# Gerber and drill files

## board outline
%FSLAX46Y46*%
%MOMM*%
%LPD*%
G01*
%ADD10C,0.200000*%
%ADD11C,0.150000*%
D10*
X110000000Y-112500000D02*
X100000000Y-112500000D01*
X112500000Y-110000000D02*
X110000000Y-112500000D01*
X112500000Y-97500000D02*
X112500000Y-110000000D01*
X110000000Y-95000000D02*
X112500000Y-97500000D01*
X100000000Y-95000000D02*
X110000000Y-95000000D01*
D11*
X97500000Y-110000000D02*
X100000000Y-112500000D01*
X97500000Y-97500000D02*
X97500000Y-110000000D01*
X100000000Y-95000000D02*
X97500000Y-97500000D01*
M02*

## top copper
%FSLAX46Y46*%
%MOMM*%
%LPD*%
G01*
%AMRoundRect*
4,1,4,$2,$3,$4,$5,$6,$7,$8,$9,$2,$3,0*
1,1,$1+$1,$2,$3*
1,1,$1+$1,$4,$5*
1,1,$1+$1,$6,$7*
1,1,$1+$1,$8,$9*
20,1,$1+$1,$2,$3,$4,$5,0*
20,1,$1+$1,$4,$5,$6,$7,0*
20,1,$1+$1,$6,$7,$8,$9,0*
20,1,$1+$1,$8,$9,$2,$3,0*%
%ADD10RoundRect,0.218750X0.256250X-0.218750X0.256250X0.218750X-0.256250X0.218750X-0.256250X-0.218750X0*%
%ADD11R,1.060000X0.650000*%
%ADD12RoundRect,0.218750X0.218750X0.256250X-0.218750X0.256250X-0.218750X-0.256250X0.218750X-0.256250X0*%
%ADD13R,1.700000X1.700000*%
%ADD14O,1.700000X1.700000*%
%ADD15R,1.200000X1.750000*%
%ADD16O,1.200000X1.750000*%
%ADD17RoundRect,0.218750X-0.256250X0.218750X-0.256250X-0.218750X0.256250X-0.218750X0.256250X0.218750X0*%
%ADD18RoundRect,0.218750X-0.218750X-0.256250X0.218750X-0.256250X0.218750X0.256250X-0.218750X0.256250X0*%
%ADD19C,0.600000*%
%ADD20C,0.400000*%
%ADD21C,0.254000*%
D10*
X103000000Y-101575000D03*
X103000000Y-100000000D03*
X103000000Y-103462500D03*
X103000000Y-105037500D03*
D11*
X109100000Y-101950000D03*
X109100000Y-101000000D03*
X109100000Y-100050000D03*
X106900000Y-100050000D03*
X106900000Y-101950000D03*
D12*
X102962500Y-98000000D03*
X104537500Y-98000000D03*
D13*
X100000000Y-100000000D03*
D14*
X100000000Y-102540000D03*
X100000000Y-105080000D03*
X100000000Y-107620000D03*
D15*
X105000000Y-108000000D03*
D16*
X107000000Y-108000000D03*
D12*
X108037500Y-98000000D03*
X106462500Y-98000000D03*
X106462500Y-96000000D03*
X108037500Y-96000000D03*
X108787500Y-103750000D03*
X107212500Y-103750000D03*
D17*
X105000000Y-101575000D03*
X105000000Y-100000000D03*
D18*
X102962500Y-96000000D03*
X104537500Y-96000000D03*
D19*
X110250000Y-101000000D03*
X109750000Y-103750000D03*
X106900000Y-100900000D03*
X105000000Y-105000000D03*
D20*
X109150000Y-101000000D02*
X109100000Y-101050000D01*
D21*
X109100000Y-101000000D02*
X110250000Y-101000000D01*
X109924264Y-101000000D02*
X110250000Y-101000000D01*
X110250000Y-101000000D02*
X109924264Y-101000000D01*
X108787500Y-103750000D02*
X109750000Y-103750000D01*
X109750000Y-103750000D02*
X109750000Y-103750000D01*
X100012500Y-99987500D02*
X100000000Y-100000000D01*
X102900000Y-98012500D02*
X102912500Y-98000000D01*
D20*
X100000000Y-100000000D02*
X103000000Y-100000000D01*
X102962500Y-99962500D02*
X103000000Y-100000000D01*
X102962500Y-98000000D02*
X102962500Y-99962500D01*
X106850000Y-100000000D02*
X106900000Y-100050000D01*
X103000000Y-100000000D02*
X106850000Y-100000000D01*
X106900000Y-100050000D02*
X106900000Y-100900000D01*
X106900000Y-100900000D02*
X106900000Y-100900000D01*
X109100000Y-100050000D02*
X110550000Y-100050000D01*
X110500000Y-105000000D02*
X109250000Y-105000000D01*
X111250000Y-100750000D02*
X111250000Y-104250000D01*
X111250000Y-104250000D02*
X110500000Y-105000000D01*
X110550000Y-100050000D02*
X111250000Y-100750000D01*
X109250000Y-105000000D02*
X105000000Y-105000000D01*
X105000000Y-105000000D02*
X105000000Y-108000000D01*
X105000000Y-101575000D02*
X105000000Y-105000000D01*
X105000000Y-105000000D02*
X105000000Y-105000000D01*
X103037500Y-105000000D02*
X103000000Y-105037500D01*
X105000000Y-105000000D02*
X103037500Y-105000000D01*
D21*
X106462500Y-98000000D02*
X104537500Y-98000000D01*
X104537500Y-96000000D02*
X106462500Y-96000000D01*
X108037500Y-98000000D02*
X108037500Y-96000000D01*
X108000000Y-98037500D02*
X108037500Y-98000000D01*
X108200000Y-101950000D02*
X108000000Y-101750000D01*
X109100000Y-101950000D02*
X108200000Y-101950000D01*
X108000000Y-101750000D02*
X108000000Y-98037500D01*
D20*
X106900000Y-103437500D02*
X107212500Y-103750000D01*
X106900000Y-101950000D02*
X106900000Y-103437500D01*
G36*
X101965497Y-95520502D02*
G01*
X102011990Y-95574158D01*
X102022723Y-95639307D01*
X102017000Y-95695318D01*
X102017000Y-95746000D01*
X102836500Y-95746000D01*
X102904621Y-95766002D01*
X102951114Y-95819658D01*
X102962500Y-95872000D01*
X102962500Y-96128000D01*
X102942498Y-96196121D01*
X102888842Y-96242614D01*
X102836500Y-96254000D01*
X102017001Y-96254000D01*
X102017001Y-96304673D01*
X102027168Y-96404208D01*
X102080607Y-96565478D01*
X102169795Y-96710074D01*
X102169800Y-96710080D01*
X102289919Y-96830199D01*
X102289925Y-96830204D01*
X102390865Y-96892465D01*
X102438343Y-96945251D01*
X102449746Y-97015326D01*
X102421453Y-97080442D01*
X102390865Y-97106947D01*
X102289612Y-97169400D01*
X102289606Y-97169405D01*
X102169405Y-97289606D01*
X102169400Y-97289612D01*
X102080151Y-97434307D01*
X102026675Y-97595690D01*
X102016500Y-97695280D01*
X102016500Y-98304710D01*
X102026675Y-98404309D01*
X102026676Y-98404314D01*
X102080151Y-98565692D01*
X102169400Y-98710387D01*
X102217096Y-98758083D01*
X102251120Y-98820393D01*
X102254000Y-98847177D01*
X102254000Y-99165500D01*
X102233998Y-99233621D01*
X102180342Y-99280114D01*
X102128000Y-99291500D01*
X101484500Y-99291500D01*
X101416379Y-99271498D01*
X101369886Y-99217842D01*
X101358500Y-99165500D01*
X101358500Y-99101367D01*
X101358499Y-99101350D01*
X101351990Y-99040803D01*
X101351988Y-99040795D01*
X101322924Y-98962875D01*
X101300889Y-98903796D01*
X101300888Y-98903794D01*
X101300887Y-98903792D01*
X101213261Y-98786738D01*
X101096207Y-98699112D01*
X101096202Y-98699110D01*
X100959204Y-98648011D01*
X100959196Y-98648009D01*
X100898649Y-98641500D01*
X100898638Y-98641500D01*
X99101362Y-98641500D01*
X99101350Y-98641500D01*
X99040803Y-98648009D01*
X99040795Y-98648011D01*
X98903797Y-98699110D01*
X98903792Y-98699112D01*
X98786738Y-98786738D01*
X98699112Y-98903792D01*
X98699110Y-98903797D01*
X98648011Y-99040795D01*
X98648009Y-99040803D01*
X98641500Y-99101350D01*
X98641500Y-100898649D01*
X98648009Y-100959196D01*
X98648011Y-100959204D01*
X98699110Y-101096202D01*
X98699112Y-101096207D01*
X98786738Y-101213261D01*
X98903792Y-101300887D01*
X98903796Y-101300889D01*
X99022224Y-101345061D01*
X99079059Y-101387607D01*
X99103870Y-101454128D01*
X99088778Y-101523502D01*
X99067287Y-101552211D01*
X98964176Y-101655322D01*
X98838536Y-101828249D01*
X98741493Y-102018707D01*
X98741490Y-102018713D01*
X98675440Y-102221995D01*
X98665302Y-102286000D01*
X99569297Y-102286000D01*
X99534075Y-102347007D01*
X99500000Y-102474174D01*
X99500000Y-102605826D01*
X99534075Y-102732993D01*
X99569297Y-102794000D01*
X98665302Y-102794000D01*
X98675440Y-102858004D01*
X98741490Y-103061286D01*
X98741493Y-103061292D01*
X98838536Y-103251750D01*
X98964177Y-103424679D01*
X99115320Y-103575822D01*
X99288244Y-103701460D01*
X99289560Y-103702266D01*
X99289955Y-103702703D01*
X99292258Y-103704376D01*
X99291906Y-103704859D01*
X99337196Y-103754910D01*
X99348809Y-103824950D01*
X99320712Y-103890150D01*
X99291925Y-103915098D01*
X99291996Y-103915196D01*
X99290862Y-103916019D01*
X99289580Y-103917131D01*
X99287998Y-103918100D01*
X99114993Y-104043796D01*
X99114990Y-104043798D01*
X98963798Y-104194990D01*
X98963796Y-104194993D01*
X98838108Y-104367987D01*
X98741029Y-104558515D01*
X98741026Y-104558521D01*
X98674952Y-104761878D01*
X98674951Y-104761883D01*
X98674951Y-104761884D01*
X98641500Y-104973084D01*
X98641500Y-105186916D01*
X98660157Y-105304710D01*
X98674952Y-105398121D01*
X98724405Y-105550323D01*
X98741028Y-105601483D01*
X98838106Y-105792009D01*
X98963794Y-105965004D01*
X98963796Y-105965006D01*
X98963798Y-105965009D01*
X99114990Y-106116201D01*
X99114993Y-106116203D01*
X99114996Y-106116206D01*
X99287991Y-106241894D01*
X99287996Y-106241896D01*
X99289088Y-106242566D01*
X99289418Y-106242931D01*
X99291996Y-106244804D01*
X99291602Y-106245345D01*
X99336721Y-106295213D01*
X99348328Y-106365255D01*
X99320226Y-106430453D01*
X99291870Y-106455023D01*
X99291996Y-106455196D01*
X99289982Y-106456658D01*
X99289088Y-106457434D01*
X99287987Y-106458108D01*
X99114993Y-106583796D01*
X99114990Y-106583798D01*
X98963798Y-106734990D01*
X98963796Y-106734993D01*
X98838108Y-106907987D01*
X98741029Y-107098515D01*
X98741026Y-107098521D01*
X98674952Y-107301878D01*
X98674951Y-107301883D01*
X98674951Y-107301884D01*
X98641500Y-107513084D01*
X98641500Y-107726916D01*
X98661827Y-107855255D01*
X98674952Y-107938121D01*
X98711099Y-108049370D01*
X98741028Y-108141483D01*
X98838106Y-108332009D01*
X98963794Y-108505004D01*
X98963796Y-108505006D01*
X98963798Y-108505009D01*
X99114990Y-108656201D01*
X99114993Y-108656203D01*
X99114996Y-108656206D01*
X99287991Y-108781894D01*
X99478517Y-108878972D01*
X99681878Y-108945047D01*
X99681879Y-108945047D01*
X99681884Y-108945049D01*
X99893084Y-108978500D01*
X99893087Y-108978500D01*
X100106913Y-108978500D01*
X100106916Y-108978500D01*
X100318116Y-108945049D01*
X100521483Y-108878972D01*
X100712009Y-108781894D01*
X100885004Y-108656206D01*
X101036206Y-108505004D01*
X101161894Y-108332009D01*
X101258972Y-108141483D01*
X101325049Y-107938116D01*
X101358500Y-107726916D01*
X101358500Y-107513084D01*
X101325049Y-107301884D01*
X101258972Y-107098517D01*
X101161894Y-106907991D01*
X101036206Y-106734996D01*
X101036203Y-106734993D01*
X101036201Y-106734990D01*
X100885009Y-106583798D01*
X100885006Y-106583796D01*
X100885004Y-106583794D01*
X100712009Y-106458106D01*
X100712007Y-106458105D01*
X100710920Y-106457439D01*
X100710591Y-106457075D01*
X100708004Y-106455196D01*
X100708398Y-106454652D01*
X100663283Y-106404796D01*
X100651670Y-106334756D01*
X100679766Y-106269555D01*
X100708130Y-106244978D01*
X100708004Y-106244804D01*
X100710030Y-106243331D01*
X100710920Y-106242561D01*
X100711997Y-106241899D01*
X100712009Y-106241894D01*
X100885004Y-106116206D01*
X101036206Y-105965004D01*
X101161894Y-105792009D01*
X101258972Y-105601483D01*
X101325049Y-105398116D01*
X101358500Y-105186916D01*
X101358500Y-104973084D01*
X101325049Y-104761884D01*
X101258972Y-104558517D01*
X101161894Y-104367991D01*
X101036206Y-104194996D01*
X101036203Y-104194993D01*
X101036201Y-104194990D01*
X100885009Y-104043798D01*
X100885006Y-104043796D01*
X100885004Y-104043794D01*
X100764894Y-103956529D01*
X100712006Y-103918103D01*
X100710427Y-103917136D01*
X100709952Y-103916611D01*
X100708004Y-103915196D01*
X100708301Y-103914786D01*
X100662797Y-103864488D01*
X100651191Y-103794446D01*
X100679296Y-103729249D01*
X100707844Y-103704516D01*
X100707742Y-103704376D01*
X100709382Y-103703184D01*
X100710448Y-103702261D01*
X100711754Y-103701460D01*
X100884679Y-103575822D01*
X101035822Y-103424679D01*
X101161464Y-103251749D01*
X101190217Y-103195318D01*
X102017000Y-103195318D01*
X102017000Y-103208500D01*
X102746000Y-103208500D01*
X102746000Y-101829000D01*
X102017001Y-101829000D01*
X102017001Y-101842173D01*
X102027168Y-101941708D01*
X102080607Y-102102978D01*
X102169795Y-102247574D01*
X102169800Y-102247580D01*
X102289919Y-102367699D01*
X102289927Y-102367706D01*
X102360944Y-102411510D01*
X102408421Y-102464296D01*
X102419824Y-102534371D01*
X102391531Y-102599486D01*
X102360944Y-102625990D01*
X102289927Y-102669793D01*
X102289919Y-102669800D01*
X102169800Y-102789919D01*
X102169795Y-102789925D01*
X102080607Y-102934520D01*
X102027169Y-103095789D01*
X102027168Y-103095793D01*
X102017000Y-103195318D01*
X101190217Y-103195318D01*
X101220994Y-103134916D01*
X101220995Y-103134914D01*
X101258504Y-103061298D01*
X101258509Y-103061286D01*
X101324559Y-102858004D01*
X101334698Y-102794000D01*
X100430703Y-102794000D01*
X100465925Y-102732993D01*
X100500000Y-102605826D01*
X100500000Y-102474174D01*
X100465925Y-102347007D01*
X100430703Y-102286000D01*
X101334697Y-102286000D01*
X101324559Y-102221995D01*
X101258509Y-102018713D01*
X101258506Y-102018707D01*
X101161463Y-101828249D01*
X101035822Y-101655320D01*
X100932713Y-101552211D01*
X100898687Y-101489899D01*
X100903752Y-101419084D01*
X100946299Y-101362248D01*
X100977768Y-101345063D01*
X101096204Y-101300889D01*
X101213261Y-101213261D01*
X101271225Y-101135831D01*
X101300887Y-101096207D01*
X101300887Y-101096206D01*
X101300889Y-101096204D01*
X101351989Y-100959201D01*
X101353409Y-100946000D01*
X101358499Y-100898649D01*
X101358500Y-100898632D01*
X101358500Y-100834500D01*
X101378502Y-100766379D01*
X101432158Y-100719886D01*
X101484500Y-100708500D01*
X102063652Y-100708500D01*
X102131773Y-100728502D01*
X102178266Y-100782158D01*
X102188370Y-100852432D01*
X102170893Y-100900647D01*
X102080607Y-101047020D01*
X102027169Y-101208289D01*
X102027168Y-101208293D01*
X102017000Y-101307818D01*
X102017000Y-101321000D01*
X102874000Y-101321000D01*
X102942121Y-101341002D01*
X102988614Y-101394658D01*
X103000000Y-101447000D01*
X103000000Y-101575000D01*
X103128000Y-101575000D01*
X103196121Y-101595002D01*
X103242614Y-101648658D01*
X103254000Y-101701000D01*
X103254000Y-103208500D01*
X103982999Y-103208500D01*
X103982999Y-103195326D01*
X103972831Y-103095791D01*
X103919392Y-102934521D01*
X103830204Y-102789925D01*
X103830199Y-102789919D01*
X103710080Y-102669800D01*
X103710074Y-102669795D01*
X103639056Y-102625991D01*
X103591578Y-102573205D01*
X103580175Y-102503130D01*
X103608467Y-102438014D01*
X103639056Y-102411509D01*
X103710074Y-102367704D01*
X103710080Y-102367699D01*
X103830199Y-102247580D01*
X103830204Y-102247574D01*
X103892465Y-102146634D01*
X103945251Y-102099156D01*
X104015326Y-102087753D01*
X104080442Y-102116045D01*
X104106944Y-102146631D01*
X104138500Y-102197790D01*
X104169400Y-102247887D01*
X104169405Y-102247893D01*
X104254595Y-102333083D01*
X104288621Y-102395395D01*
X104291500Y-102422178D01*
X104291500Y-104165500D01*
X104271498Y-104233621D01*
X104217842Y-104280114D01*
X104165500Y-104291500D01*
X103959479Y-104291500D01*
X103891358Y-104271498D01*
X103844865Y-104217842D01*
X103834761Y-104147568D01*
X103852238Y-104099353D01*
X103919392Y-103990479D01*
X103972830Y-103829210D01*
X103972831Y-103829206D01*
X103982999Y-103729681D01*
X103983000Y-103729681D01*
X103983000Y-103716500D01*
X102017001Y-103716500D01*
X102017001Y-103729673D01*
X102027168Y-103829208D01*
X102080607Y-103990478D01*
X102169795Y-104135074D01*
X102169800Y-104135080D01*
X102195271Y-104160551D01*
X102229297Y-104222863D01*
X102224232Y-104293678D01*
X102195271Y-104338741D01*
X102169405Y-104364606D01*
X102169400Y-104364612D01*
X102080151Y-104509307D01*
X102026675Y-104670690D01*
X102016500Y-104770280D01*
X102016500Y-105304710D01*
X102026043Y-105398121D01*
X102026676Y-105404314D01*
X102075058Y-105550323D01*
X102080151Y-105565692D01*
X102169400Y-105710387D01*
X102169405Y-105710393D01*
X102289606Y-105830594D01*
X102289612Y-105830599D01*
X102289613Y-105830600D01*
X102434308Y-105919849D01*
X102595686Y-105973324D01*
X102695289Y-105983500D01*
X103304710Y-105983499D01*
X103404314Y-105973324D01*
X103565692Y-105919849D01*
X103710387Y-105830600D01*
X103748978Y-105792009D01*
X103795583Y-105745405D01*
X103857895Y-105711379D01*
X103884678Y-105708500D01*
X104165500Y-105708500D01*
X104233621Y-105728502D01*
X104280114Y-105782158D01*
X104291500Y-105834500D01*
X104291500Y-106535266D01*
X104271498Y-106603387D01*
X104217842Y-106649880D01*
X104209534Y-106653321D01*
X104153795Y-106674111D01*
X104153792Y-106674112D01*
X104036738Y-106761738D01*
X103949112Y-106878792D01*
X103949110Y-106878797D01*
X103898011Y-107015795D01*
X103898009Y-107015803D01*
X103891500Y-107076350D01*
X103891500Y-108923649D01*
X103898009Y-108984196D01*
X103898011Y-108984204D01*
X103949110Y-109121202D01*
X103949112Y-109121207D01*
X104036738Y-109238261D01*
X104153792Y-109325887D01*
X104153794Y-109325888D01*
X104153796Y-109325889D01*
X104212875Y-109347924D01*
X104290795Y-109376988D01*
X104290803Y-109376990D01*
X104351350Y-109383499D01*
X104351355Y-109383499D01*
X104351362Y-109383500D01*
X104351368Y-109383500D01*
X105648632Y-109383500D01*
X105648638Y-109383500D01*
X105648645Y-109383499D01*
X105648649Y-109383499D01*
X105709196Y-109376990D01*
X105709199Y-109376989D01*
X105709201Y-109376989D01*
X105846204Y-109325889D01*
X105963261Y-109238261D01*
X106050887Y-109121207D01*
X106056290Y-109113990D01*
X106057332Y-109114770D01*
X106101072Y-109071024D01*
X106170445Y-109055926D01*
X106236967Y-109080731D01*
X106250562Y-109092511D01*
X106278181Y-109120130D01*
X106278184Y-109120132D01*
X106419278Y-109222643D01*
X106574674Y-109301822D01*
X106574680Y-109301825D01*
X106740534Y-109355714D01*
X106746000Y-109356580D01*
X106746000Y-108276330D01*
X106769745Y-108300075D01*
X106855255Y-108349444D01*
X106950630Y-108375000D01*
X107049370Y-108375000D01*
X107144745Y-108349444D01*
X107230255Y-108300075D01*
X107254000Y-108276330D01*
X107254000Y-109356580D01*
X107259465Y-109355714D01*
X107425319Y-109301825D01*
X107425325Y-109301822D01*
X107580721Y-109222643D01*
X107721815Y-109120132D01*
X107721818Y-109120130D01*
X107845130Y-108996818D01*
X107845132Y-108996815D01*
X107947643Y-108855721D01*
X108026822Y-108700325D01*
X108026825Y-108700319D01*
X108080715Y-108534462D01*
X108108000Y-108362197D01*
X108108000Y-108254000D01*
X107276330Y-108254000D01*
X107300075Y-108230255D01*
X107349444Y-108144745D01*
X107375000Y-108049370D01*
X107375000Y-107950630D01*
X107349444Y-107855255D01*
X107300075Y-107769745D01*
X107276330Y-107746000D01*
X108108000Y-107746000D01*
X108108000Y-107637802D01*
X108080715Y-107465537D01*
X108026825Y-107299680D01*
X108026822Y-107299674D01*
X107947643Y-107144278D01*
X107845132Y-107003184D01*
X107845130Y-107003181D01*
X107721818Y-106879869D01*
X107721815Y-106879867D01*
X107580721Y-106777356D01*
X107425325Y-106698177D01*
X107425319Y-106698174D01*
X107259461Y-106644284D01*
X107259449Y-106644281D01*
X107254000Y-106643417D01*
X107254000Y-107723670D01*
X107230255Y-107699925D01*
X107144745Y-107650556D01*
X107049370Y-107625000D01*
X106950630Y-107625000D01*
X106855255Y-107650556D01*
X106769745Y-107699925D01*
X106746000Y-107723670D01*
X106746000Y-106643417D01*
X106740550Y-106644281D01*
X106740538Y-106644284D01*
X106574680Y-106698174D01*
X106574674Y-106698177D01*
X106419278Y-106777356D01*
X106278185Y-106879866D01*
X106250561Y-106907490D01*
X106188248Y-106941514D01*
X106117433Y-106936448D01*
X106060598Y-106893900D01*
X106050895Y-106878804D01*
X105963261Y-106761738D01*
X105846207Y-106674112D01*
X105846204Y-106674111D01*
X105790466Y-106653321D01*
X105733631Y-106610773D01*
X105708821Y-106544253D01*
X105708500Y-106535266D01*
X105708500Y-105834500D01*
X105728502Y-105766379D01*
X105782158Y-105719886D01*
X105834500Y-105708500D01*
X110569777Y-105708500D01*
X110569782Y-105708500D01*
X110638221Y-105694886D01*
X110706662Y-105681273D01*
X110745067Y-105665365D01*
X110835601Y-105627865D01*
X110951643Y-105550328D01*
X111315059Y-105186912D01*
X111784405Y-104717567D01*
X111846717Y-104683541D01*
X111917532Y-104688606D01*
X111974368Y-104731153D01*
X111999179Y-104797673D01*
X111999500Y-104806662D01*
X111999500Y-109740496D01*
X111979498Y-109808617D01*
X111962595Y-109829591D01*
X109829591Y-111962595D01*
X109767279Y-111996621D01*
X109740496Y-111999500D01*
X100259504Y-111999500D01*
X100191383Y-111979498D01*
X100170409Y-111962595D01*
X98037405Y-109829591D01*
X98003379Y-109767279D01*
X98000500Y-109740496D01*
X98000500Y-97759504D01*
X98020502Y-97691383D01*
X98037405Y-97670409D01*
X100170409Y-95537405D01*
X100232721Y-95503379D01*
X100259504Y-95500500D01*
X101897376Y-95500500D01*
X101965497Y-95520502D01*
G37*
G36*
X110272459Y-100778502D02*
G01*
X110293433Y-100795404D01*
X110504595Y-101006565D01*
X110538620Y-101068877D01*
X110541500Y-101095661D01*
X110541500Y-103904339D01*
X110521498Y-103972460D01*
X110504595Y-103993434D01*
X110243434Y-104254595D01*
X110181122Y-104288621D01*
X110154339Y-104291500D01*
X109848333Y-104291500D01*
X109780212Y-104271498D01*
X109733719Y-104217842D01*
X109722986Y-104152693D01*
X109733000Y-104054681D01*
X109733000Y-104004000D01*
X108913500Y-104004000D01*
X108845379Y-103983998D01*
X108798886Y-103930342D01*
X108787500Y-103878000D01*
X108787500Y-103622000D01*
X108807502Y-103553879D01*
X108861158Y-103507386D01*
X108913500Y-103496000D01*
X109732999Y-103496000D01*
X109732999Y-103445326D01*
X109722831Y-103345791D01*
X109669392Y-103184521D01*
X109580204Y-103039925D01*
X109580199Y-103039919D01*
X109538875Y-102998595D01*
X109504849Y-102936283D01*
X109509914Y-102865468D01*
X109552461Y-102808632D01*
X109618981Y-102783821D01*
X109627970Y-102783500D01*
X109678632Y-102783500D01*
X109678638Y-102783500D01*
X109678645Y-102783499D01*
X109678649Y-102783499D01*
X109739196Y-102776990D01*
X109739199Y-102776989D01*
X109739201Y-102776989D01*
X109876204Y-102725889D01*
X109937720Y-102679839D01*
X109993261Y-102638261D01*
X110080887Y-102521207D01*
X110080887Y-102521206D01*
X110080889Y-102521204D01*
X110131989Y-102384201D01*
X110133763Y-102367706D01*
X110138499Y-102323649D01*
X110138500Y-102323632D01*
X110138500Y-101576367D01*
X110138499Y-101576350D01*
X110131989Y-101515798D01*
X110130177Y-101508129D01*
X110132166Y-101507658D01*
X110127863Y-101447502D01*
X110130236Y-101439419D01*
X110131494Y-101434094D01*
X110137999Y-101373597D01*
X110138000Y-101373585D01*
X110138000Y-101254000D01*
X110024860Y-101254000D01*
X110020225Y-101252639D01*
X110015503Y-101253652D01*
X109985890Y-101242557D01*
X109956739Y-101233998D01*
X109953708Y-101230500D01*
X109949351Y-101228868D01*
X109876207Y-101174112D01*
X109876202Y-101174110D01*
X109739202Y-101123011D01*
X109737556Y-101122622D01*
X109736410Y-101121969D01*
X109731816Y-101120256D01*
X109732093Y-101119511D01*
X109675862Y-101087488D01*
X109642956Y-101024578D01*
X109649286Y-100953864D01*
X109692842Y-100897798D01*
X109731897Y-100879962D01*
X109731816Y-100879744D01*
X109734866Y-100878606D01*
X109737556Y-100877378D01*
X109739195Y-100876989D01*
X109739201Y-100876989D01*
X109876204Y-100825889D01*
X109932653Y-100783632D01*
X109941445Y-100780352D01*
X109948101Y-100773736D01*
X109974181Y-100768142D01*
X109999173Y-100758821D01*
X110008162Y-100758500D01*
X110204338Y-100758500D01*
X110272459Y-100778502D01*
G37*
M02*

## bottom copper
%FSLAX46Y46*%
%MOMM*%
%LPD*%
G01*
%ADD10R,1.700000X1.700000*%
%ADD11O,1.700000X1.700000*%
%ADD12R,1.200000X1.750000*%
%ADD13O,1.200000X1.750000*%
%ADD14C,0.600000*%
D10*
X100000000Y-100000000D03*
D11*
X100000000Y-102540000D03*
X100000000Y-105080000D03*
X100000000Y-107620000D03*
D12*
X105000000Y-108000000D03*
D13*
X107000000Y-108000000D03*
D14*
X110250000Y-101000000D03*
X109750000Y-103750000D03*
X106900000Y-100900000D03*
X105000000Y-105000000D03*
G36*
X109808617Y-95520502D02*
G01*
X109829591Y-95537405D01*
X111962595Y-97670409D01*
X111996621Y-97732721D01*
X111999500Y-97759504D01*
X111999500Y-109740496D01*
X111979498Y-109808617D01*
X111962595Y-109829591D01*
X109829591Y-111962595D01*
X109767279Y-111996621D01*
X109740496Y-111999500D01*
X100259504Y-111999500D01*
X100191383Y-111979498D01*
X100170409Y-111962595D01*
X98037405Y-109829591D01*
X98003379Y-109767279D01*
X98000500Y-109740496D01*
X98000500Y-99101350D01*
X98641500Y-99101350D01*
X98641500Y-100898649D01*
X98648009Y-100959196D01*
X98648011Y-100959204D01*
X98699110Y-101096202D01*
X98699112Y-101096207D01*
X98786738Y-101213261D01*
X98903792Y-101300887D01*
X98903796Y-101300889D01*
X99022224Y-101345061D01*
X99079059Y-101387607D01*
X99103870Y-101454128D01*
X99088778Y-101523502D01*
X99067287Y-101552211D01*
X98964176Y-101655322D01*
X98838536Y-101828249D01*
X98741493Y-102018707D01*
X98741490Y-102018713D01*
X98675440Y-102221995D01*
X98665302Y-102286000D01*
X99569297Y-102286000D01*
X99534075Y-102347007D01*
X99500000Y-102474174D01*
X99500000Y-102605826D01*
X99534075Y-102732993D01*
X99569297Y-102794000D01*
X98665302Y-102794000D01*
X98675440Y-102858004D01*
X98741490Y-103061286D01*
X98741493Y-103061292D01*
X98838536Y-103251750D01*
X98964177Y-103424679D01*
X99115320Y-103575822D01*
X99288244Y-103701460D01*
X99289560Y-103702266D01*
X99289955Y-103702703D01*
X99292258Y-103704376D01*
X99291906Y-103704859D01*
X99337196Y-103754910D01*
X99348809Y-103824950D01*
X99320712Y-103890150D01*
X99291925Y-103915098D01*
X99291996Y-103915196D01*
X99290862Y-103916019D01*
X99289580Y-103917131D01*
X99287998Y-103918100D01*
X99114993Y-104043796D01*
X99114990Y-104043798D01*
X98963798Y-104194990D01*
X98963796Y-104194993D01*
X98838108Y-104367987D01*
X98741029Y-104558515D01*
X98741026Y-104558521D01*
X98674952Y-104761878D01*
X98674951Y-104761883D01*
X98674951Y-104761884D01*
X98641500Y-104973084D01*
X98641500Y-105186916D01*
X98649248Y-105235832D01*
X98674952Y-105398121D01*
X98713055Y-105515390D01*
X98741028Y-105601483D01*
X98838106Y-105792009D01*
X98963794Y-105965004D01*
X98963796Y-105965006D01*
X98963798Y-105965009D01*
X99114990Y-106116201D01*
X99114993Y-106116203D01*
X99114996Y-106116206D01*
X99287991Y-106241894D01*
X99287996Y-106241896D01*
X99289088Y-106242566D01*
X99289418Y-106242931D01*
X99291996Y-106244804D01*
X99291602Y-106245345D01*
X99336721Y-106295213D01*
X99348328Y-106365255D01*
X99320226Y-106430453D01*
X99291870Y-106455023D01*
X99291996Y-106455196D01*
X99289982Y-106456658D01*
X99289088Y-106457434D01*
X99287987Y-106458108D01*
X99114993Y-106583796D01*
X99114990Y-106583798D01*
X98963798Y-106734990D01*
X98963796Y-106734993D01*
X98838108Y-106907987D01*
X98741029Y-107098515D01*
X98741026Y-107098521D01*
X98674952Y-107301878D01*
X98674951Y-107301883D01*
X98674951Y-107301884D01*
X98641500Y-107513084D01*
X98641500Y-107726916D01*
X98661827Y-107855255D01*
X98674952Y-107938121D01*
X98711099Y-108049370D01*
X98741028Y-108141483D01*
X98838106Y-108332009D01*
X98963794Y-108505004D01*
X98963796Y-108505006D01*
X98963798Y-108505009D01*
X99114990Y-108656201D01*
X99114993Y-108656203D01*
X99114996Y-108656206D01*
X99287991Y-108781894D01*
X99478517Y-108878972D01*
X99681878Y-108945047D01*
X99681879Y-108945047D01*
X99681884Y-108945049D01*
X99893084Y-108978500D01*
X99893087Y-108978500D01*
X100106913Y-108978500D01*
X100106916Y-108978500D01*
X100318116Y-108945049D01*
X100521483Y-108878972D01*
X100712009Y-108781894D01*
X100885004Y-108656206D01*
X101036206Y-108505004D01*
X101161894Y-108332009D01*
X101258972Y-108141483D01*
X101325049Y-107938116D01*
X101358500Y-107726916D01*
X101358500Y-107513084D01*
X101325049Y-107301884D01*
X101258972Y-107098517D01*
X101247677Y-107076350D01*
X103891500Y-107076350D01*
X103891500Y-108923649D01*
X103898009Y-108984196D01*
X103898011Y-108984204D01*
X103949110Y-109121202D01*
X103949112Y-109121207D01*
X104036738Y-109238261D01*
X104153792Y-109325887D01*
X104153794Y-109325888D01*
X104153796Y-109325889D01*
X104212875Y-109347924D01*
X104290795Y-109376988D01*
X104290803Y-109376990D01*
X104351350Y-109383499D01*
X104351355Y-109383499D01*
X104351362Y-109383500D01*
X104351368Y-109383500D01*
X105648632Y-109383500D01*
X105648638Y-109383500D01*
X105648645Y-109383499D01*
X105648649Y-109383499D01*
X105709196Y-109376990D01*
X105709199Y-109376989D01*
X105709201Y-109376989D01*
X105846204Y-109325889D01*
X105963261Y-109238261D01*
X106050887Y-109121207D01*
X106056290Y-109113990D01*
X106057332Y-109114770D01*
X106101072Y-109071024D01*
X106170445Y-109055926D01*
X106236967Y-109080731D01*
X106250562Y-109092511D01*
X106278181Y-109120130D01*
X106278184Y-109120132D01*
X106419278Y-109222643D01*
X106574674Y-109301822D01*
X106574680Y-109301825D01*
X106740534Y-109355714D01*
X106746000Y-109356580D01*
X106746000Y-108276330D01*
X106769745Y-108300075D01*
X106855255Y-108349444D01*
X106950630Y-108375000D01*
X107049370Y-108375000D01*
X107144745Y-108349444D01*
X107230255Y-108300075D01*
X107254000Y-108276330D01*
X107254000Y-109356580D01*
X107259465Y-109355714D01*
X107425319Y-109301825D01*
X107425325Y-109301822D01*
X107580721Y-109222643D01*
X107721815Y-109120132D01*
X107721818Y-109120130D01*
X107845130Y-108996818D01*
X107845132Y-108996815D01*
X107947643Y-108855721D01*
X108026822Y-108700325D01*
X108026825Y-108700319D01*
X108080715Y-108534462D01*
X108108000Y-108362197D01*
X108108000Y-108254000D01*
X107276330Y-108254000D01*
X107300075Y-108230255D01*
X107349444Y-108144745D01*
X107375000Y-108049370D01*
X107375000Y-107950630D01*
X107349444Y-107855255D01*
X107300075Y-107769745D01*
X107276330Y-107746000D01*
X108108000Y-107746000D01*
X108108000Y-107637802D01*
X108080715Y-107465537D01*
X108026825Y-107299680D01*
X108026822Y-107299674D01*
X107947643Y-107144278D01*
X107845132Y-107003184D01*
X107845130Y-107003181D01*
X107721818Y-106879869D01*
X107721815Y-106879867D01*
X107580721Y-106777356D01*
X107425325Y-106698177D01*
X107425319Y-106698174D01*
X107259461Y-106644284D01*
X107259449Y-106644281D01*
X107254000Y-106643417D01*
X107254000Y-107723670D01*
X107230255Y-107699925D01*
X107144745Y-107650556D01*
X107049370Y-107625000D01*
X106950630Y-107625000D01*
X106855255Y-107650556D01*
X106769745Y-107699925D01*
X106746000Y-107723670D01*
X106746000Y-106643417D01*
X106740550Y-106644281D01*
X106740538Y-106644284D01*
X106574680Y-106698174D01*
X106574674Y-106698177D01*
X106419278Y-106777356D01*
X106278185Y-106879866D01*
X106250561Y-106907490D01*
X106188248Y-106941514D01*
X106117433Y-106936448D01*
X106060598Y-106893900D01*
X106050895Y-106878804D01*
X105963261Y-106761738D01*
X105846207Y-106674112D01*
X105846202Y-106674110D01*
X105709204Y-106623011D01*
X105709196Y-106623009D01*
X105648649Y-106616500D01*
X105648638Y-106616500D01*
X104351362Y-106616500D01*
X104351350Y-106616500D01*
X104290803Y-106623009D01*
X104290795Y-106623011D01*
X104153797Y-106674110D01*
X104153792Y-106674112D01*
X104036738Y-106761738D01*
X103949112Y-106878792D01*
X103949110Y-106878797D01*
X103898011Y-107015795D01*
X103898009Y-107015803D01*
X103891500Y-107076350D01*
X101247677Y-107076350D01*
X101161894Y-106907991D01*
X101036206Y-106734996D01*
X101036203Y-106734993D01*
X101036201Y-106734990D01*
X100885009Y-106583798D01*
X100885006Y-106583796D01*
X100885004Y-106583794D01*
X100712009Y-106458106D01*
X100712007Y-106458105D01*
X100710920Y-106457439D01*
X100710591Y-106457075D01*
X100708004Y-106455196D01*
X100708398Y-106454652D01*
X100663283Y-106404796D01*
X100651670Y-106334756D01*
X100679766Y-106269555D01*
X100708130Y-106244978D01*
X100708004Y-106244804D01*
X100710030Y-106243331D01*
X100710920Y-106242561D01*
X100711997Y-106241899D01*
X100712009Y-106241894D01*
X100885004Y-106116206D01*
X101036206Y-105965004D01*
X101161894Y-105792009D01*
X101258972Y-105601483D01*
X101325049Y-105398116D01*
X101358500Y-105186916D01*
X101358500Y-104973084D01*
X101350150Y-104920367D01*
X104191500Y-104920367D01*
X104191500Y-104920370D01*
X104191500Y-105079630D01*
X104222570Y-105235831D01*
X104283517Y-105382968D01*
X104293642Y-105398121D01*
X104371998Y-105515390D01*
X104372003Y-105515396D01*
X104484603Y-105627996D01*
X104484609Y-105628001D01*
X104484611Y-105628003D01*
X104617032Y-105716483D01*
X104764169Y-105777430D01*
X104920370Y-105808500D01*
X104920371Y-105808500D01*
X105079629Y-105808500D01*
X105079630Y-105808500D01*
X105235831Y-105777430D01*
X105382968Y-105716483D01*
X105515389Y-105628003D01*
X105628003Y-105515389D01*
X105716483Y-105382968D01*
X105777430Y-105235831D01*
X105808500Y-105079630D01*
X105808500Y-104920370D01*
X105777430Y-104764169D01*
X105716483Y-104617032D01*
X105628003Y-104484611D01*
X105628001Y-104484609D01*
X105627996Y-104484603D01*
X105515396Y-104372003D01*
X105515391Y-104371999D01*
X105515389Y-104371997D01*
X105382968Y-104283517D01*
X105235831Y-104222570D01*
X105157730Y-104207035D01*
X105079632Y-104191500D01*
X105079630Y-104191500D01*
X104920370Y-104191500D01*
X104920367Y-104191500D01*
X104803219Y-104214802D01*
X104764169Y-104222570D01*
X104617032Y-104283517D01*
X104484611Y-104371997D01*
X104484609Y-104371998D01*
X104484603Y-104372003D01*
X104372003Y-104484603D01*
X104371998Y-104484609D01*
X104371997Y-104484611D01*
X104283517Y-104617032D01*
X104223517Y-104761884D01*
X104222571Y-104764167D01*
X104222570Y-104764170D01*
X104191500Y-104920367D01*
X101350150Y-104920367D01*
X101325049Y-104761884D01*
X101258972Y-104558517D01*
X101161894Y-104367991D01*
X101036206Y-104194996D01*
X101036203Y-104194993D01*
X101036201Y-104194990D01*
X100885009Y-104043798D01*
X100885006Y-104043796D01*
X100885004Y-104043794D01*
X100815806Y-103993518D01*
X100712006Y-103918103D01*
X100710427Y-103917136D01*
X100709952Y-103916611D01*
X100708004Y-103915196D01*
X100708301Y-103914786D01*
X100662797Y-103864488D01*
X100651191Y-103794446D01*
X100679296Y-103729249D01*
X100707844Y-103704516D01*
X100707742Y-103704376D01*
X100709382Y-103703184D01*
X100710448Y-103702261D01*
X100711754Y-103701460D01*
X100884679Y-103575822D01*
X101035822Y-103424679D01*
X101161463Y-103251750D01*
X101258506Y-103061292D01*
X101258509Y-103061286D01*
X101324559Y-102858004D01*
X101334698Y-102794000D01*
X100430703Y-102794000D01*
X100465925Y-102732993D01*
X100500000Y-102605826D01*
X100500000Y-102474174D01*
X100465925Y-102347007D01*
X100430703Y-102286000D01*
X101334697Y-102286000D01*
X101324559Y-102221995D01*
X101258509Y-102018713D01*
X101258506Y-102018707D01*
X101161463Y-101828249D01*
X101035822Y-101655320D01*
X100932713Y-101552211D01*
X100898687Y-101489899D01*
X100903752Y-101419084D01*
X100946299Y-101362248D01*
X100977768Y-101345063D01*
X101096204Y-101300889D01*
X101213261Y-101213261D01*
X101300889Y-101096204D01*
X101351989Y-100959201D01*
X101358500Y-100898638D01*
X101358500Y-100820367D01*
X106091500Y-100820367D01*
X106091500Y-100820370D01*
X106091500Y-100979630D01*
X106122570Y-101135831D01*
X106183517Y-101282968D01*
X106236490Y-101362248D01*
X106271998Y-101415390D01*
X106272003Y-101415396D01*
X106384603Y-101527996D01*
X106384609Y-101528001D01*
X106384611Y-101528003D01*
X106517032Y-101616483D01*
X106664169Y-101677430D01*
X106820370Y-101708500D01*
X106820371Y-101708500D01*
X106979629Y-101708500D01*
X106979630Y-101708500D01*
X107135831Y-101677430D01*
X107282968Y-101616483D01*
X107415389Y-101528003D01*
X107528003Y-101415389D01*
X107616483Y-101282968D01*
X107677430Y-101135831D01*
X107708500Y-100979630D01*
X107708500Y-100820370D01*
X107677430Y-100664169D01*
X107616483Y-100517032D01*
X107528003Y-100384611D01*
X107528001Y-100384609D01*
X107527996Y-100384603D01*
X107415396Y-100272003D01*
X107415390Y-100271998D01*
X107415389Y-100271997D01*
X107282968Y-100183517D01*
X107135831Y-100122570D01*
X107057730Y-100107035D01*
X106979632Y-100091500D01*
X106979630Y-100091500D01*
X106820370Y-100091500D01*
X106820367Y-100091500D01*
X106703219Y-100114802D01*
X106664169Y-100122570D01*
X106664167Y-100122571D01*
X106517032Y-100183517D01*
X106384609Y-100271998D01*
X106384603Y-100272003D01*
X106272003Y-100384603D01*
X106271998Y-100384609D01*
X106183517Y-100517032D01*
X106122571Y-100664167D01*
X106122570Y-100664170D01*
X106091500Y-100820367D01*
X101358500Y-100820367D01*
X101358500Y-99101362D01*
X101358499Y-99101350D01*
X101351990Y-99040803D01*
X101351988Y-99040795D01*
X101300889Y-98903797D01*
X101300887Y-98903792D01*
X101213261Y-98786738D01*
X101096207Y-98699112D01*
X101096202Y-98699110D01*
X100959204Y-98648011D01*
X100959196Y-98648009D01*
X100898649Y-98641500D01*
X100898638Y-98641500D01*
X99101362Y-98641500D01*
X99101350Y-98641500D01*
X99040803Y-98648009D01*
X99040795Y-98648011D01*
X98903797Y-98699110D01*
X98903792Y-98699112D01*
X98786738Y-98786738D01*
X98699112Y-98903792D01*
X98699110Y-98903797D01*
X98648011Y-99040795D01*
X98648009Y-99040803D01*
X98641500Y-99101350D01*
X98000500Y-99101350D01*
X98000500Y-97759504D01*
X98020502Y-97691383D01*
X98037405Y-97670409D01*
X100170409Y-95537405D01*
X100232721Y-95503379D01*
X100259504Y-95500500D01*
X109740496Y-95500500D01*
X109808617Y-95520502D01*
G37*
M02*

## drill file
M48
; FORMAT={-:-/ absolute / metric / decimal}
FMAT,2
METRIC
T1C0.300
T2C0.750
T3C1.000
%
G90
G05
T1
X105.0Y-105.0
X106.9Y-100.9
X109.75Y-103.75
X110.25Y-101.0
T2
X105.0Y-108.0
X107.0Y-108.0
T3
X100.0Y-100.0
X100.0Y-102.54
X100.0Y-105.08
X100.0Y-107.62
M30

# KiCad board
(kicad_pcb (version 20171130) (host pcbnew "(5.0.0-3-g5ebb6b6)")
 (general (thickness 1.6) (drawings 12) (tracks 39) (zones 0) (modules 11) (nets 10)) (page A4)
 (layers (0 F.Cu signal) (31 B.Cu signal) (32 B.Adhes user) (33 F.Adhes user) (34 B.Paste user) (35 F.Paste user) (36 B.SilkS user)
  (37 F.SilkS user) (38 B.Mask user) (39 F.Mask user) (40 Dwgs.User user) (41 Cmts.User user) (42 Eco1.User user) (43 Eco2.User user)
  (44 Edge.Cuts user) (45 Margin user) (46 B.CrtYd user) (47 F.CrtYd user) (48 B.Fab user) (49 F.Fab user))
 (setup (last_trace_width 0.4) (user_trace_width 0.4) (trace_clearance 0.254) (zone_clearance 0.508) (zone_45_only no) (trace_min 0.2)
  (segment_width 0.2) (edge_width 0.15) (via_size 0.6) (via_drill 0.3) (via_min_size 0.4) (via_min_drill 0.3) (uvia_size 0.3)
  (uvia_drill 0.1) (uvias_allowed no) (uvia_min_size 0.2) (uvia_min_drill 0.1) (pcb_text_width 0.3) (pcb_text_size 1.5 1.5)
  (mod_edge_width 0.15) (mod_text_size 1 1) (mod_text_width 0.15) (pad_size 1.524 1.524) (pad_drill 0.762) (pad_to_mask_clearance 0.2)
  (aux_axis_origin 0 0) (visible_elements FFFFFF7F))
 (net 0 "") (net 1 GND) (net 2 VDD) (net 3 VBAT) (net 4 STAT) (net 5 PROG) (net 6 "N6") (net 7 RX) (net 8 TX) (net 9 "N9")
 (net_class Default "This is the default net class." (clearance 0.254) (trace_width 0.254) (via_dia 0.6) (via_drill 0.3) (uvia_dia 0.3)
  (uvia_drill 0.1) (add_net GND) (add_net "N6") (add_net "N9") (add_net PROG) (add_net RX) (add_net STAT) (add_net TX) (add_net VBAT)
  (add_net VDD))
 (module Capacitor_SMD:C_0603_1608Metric (layer F.Cu) (at 103 100.7875 90)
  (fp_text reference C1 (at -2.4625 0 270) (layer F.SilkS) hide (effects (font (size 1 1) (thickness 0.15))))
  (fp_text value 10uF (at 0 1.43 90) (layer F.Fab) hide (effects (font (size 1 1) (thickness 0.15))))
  (pad 1 smd roundrect (at -0.7875 0 90) (size 0.875 0.95) (layers F.Cu F.Paste F.Mask) (roundrect_rratio 0.25) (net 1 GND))
  (pad 2 smd roundrect (at 0.7875 0 90) (size 0.875 0.95) (layers F.Cu F.Paste F.Mask) (roundrect_rratio 0.25) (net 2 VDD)))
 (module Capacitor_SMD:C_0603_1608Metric (layer F.Cu) (at 103 104.25 90)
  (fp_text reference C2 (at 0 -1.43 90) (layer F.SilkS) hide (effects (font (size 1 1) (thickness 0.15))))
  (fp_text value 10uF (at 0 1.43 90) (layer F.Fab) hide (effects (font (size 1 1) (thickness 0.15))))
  (pad 2 smd roundrect (at 0.7875 0 90) (size 0.875 0.95) (layers F.Cu F.Paste F.Mask) (roundrect_rratio 0.25) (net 1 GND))
  (pad 1 smd roundrect (at -0.7875 0 90) (size 0.875 0.95) (layers F.Cu F.Paste F.Mask) (roundrect_rratio 0.25) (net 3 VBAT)))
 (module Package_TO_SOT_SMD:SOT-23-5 (layer F.Cu) (at 108 101 180)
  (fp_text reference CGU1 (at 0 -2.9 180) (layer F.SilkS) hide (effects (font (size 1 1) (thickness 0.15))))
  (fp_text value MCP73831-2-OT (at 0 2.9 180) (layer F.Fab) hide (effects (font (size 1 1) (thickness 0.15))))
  (pad 1 smd rect (at -1.1 -0.95 180) (size 1.06 0.65) (layers F.Cu F.Paste F.Mask) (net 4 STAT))
  (pad 2 smd rect (at -1.1 0 180) (size 1.06 0.65) (layers F.Cu F.Paste F.Mask) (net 1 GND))
  (pad 3 smd rect (at -1.1 0.95 180) (size 1.06 0.65) (layers F.Cu F.Paste F.Mask) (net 3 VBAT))
  (pad 4 smd rect (at 1.1 0.95 180) (size 1.06 0.65) (layers F.Cu F.Paste F.Mask) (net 2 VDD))
  (pad 5 smd rect (at 1.1 -0.95 180) (size 1.06 0.65) (layers F.Cu F.Paste F.Mask) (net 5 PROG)))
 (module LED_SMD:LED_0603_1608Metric (layer F.Cu) (at 103.75 98 180)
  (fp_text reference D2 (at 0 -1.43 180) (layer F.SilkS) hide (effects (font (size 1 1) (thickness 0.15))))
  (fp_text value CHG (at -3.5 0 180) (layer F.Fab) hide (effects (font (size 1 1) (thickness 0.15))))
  (pad 2 smd roundrect (at 0.7875 0 180) (size 0.875 0.95) (layers F.Cu F.Paste F.Mask) (roundrect_rratio 0.25) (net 2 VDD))
  (pad 1 smd roundrect (at -0.7875 0 180) (size 0.875 0.95) (layers F.Cu F.Paste F.Mask) (roundrect_rratio 0.25) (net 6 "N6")))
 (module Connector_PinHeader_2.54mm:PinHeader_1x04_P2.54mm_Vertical (layer F.Cu) (at 100 100)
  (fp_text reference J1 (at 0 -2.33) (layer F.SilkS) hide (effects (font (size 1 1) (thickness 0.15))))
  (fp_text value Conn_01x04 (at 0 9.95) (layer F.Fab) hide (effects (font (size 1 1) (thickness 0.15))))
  (pad 1 thru_hole rect (at 0 0) (size 1.7 1.7) (drill 1) (layers *.Cu *.Mask) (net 2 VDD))
  (pad 2 thru_hole oval (at 0 2.54) (size 1.7 1.7) (drill 1) (layers *.Cu *.Mask) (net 1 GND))
  (pad 3 thru_hole oval (at 0 5.08) (size 1.7 1.7) (drill 1) (layers *.Cu *.Mask) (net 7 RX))
  (pad 4 thru_hole oval (at 0 7.62) (size 1.7 1.7) (drill 1) (layers *.Cu *.Mask) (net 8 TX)))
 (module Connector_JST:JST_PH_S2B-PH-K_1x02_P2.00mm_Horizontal (layer F.Cu) (at 105 108)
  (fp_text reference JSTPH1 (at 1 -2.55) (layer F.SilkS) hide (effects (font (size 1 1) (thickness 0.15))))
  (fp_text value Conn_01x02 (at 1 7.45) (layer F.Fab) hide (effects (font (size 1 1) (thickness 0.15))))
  (pad 1 thru_hole rect (at 0 0) (size 1.2 1.75) (drill 0.75) (layers *.Cu *.Mask) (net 3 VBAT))
  (pad 2 thru_hole oval (at 2 0) (size 1.2 1.75) (drill 0.75) (layers *.Cu *.Mask) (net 1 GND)))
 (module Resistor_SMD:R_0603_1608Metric (layer F.Cu) (at 107.25 98 180)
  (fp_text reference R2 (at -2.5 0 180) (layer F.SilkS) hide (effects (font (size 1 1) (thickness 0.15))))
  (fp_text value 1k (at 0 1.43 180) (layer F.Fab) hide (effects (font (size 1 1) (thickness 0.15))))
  (pad 1 smd roundrect (at -0.7875 0 180) (size 0.875 0.95) (layers F.Cu F.Paste F.Mask) (roundrect_rratio 0.25) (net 4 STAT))
  (pad 2 smd roundrect (at 0.7875 0 180) (size 0.875 0.95) (layers F.Cu F.Paste F.Mask) (roundrect_rratio 0.25) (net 6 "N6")))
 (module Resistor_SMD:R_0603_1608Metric (layer F.Cu) (at 107.25 96 180)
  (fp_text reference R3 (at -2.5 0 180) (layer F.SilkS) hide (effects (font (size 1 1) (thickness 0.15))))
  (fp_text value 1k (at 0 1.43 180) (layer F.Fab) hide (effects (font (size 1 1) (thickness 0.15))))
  (pad 2 smd roundrect (at 0.7875 0 180) (size 0.875 0.95) (layers F.Cu F.Paste F.Mask) (roundrect_rratio 0.25) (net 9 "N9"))
  (pad 1 smd roundrect (at -0.7875 0 180) (size 0.875 0.95) (layers F.Cu F.Paste F.Mask) (roundrect_rratio 0.25) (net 4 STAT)))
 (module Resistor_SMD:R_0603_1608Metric (layer F.Cu) (at 108 103.75 180)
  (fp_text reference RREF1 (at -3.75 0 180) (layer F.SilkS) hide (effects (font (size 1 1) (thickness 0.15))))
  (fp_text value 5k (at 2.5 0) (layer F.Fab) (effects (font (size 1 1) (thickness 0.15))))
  (pad 1 smd roundrect (at -0.7875 0 180) (size 0.875 0.95) (layers F.Cu F.Paste F.Mask) (roundrect_rratio 0.25) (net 1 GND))
  (pad 2 smd roundrect (at 0.7875 0 180) (size 0.875 0.95) (layers F.Cu F.Paste F.Mask) (roundrect_rratio 0.25) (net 5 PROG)))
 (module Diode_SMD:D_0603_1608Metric (layer F.Cu) (at 105 100.7875 270)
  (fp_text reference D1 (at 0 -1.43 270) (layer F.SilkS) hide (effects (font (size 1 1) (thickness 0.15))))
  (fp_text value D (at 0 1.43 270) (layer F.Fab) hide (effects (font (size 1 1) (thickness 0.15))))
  (pad 2 smd roundrect (at 0.7875 0 270) (size 0.875 0.95) (layers F.Cu F.Paste F.Mask) (roundrect_rratio 0.25) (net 3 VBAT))
  (pad 1 smd roundrect (at -0.7875 0 270) (size 0.875 0.95) (layers F.Cu F.Paste F.Mask) (roundrect_rratio 0.25) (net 2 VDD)))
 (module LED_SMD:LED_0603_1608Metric (layer F.Cu) (at 103.75 96)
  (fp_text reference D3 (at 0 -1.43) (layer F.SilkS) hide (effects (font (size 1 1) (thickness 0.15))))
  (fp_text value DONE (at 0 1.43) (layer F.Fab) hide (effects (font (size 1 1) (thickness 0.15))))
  (pad 1 smd roundrect (at -0.7875 0) (size 0.875 0.95) (layers F.Cu F.Paste F.Mask) (roundrect_rratio 0.25) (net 1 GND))
  (pad 2 smd roundrect (at 0.7875 0) (size 0.875 0.95) (layers F.Cu F.Paste F.Mask) (roundrect_rratio 0.25) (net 9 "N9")))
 (gr_line (start 110 112.5) (end 100 112.5) (layer Edge.Cuts) (width 0.2))
 (gr_line (start 112.5 110) (end 110 112.5) (layer Edge.Cuts) (width 0.2))
 (gr_line (start 112.5 97.5) (end 112.5 110) (layer Edge.Cuts) (width 0.2))
 (gr_line (start 110 95) (end 112.5 97.5) (layer Edge.Cuts) (width 0.2))
 (gr_line (start 100 95) (end 110 95) (layer Edge.Cuts) (width 0.2))
 (gr_line (start 97.5 110) (end 100 112.5) (layer Edge.Cuts) (width 0.15))
 (gr_line (start 97.5 97.5) (end 97.5 110) (layer Edge.Cuts) (width 0.15))
 (gr_line (start 100 95) (end 97.5 97.5) (layer Edge.Cuts) (width 0.15))
 (segment (start 109.15 101) (end 109.1 101.05) (width 0.4) (layer F.Cu) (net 1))
 (segment (start 109.1 101) (end 110.25 101) (width 0.254) (layer F.Cu) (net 1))
 (segment (start 109.924264 101) (end 110.25 101) (width 0.254) (layer F.Cu) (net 1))
 (segment (start 110.25 101) (end 109.924264 101) (width 0.254) (layer F.Cu) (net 1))
 (via (at 110.25 101) (size 0.6) (drill 0.3) (layers F.Cu B.Cu) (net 1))
 (segment (start 108.7875 103.75) (end 109.75 103.75) (width 0.254) (layer F.Cu) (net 1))
 (segment (start 109.75 103.75) (end 109.75 103.75) (width 0.254) (layer F.Cu) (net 1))
 (via (at 109.75 103.75) (size 0.6) (drill 0.3) (layers F.Cu B.Cu) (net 1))
 (segment (start 100.0125 99.9875) (end 100 100) (width 0.254) (layer F.Cu) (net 2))
 (segment (start 102.9 98.0125) (end 102.9125 98) (width 0.254) (layer F.Cu) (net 2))
 (segment (start 100 100) (end 103 100) (width 0.4) (layer F.Cu) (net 2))
 (segment (start 102.9625 99.9625) (end 103 100) (width 0.4) (layer F.Cu) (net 2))
 (segment (start 102.9625 98) (end 102.9625 99.9625) (width 0.4) (layer F.Cu) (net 2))
 (segment (start 106.85 100) (end 106.9 100.05) (width 0.4) (layer F.Cu) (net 2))
 (segment (start 103 100) (end 106.85 100) (width 0.4) (layer F.Cu) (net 2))
 (segment (start 106.9 100.05) (end 106.9 100.9) (width 0.4) (layer F.Cu) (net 2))
 (segment (start 106.9 100.9) (end 106.9 100.9) (width 0.4) (layer F.Cu) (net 2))
 (via (at 106.9 100.9) (size 0.6) (drill 0.3) (layers F.Cu B.Cu) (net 2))
 (segment (start 109.1 100.05) (end 110.55 100.05) (width 0.4) (layer F.Cu) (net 3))
 (segment (start 110.5 105) (end 109.25 105) (width 0.4) (layer F.Cu) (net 3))
 (segment (start 111.25 100.75) (end 111.25 104.25) (width 0.4) (layer F.Cu) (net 3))
 (segment (start 111.25 104.25) (end 110.5 105) (width 0.4) (layer F.Cu) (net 3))
 (segment (start 110.55 100.05) (end 111.25 100.75) (width 0.4) (layer F.Cu) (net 3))
 (segment (start 109.25 105) (end 105 105) (width 0.4) (layer F.Cu) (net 3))
 (segment (start 105 105) (end 105 108) (width 0.4) (layer F.Cu) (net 3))
 (segment (start 105 101.575) (end 105 105) (width 0.4) (layer F.Cu) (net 3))
 (segment (start 105 105) (end 105 105) (width 0.4) (layer F.Cu) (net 3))
 (via (at 105 105) (size 0.6) (drill 0.3) (layers F.Cu B.Cu) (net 3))
 (segment (start 103.0375 105) (end 103 105.0375) (width 0.4) (layer F.Cu) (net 3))
 (segment (start 105 105) (end 103.0375 105) (width 0.4) (layer F.Cu) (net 3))
 (segment (start 106.4625 98) (end 104.5375 98) (width 0.254) (layer F.Cu) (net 6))
 (segment (start 104.5375 96) (end 106.4625 96) (width 0.254) (layer F.Cu) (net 9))
 (segment (start 108.0375 98) (end 108.0375 96) (width 0.254) (layer F.Cu) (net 4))
 (segment (start 108 98.0375) (end 108.0375 98) (width 0.254) (layer F.Cu) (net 4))
 (segment (start 108.2 101.95) (end 108 101.75) (width 0.254) (layer F.Cu) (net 4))
 (segment (start 109.1 101.95) (end 108.2 101.95) (width 0.254) (layer F.Cu) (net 4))
 (segment (start 108 101.75) (end 108 98.0375) (width 0.254) (layer F.Cu) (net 4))
 (segment (start 106.9 103.4375) (end 107.2125 103.75) (width 0.4) (layer F.Cu) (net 5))
 (segment (start 106.9 101.95) (end 106.9 103.4375) (width 0.4) (layer F.Cu) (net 5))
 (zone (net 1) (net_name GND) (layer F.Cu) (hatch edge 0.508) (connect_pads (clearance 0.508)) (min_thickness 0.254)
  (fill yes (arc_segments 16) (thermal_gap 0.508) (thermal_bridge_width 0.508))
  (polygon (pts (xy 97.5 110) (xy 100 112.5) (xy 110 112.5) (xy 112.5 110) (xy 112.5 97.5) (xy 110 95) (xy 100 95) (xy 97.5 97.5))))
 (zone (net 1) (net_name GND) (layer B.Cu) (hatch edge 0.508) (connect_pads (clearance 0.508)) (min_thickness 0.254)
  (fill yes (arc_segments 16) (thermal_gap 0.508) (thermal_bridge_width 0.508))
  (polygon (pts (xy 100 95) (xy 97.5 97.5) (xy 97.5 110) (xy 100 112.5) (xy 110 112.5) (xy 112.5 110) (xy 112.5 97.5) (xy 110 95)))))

